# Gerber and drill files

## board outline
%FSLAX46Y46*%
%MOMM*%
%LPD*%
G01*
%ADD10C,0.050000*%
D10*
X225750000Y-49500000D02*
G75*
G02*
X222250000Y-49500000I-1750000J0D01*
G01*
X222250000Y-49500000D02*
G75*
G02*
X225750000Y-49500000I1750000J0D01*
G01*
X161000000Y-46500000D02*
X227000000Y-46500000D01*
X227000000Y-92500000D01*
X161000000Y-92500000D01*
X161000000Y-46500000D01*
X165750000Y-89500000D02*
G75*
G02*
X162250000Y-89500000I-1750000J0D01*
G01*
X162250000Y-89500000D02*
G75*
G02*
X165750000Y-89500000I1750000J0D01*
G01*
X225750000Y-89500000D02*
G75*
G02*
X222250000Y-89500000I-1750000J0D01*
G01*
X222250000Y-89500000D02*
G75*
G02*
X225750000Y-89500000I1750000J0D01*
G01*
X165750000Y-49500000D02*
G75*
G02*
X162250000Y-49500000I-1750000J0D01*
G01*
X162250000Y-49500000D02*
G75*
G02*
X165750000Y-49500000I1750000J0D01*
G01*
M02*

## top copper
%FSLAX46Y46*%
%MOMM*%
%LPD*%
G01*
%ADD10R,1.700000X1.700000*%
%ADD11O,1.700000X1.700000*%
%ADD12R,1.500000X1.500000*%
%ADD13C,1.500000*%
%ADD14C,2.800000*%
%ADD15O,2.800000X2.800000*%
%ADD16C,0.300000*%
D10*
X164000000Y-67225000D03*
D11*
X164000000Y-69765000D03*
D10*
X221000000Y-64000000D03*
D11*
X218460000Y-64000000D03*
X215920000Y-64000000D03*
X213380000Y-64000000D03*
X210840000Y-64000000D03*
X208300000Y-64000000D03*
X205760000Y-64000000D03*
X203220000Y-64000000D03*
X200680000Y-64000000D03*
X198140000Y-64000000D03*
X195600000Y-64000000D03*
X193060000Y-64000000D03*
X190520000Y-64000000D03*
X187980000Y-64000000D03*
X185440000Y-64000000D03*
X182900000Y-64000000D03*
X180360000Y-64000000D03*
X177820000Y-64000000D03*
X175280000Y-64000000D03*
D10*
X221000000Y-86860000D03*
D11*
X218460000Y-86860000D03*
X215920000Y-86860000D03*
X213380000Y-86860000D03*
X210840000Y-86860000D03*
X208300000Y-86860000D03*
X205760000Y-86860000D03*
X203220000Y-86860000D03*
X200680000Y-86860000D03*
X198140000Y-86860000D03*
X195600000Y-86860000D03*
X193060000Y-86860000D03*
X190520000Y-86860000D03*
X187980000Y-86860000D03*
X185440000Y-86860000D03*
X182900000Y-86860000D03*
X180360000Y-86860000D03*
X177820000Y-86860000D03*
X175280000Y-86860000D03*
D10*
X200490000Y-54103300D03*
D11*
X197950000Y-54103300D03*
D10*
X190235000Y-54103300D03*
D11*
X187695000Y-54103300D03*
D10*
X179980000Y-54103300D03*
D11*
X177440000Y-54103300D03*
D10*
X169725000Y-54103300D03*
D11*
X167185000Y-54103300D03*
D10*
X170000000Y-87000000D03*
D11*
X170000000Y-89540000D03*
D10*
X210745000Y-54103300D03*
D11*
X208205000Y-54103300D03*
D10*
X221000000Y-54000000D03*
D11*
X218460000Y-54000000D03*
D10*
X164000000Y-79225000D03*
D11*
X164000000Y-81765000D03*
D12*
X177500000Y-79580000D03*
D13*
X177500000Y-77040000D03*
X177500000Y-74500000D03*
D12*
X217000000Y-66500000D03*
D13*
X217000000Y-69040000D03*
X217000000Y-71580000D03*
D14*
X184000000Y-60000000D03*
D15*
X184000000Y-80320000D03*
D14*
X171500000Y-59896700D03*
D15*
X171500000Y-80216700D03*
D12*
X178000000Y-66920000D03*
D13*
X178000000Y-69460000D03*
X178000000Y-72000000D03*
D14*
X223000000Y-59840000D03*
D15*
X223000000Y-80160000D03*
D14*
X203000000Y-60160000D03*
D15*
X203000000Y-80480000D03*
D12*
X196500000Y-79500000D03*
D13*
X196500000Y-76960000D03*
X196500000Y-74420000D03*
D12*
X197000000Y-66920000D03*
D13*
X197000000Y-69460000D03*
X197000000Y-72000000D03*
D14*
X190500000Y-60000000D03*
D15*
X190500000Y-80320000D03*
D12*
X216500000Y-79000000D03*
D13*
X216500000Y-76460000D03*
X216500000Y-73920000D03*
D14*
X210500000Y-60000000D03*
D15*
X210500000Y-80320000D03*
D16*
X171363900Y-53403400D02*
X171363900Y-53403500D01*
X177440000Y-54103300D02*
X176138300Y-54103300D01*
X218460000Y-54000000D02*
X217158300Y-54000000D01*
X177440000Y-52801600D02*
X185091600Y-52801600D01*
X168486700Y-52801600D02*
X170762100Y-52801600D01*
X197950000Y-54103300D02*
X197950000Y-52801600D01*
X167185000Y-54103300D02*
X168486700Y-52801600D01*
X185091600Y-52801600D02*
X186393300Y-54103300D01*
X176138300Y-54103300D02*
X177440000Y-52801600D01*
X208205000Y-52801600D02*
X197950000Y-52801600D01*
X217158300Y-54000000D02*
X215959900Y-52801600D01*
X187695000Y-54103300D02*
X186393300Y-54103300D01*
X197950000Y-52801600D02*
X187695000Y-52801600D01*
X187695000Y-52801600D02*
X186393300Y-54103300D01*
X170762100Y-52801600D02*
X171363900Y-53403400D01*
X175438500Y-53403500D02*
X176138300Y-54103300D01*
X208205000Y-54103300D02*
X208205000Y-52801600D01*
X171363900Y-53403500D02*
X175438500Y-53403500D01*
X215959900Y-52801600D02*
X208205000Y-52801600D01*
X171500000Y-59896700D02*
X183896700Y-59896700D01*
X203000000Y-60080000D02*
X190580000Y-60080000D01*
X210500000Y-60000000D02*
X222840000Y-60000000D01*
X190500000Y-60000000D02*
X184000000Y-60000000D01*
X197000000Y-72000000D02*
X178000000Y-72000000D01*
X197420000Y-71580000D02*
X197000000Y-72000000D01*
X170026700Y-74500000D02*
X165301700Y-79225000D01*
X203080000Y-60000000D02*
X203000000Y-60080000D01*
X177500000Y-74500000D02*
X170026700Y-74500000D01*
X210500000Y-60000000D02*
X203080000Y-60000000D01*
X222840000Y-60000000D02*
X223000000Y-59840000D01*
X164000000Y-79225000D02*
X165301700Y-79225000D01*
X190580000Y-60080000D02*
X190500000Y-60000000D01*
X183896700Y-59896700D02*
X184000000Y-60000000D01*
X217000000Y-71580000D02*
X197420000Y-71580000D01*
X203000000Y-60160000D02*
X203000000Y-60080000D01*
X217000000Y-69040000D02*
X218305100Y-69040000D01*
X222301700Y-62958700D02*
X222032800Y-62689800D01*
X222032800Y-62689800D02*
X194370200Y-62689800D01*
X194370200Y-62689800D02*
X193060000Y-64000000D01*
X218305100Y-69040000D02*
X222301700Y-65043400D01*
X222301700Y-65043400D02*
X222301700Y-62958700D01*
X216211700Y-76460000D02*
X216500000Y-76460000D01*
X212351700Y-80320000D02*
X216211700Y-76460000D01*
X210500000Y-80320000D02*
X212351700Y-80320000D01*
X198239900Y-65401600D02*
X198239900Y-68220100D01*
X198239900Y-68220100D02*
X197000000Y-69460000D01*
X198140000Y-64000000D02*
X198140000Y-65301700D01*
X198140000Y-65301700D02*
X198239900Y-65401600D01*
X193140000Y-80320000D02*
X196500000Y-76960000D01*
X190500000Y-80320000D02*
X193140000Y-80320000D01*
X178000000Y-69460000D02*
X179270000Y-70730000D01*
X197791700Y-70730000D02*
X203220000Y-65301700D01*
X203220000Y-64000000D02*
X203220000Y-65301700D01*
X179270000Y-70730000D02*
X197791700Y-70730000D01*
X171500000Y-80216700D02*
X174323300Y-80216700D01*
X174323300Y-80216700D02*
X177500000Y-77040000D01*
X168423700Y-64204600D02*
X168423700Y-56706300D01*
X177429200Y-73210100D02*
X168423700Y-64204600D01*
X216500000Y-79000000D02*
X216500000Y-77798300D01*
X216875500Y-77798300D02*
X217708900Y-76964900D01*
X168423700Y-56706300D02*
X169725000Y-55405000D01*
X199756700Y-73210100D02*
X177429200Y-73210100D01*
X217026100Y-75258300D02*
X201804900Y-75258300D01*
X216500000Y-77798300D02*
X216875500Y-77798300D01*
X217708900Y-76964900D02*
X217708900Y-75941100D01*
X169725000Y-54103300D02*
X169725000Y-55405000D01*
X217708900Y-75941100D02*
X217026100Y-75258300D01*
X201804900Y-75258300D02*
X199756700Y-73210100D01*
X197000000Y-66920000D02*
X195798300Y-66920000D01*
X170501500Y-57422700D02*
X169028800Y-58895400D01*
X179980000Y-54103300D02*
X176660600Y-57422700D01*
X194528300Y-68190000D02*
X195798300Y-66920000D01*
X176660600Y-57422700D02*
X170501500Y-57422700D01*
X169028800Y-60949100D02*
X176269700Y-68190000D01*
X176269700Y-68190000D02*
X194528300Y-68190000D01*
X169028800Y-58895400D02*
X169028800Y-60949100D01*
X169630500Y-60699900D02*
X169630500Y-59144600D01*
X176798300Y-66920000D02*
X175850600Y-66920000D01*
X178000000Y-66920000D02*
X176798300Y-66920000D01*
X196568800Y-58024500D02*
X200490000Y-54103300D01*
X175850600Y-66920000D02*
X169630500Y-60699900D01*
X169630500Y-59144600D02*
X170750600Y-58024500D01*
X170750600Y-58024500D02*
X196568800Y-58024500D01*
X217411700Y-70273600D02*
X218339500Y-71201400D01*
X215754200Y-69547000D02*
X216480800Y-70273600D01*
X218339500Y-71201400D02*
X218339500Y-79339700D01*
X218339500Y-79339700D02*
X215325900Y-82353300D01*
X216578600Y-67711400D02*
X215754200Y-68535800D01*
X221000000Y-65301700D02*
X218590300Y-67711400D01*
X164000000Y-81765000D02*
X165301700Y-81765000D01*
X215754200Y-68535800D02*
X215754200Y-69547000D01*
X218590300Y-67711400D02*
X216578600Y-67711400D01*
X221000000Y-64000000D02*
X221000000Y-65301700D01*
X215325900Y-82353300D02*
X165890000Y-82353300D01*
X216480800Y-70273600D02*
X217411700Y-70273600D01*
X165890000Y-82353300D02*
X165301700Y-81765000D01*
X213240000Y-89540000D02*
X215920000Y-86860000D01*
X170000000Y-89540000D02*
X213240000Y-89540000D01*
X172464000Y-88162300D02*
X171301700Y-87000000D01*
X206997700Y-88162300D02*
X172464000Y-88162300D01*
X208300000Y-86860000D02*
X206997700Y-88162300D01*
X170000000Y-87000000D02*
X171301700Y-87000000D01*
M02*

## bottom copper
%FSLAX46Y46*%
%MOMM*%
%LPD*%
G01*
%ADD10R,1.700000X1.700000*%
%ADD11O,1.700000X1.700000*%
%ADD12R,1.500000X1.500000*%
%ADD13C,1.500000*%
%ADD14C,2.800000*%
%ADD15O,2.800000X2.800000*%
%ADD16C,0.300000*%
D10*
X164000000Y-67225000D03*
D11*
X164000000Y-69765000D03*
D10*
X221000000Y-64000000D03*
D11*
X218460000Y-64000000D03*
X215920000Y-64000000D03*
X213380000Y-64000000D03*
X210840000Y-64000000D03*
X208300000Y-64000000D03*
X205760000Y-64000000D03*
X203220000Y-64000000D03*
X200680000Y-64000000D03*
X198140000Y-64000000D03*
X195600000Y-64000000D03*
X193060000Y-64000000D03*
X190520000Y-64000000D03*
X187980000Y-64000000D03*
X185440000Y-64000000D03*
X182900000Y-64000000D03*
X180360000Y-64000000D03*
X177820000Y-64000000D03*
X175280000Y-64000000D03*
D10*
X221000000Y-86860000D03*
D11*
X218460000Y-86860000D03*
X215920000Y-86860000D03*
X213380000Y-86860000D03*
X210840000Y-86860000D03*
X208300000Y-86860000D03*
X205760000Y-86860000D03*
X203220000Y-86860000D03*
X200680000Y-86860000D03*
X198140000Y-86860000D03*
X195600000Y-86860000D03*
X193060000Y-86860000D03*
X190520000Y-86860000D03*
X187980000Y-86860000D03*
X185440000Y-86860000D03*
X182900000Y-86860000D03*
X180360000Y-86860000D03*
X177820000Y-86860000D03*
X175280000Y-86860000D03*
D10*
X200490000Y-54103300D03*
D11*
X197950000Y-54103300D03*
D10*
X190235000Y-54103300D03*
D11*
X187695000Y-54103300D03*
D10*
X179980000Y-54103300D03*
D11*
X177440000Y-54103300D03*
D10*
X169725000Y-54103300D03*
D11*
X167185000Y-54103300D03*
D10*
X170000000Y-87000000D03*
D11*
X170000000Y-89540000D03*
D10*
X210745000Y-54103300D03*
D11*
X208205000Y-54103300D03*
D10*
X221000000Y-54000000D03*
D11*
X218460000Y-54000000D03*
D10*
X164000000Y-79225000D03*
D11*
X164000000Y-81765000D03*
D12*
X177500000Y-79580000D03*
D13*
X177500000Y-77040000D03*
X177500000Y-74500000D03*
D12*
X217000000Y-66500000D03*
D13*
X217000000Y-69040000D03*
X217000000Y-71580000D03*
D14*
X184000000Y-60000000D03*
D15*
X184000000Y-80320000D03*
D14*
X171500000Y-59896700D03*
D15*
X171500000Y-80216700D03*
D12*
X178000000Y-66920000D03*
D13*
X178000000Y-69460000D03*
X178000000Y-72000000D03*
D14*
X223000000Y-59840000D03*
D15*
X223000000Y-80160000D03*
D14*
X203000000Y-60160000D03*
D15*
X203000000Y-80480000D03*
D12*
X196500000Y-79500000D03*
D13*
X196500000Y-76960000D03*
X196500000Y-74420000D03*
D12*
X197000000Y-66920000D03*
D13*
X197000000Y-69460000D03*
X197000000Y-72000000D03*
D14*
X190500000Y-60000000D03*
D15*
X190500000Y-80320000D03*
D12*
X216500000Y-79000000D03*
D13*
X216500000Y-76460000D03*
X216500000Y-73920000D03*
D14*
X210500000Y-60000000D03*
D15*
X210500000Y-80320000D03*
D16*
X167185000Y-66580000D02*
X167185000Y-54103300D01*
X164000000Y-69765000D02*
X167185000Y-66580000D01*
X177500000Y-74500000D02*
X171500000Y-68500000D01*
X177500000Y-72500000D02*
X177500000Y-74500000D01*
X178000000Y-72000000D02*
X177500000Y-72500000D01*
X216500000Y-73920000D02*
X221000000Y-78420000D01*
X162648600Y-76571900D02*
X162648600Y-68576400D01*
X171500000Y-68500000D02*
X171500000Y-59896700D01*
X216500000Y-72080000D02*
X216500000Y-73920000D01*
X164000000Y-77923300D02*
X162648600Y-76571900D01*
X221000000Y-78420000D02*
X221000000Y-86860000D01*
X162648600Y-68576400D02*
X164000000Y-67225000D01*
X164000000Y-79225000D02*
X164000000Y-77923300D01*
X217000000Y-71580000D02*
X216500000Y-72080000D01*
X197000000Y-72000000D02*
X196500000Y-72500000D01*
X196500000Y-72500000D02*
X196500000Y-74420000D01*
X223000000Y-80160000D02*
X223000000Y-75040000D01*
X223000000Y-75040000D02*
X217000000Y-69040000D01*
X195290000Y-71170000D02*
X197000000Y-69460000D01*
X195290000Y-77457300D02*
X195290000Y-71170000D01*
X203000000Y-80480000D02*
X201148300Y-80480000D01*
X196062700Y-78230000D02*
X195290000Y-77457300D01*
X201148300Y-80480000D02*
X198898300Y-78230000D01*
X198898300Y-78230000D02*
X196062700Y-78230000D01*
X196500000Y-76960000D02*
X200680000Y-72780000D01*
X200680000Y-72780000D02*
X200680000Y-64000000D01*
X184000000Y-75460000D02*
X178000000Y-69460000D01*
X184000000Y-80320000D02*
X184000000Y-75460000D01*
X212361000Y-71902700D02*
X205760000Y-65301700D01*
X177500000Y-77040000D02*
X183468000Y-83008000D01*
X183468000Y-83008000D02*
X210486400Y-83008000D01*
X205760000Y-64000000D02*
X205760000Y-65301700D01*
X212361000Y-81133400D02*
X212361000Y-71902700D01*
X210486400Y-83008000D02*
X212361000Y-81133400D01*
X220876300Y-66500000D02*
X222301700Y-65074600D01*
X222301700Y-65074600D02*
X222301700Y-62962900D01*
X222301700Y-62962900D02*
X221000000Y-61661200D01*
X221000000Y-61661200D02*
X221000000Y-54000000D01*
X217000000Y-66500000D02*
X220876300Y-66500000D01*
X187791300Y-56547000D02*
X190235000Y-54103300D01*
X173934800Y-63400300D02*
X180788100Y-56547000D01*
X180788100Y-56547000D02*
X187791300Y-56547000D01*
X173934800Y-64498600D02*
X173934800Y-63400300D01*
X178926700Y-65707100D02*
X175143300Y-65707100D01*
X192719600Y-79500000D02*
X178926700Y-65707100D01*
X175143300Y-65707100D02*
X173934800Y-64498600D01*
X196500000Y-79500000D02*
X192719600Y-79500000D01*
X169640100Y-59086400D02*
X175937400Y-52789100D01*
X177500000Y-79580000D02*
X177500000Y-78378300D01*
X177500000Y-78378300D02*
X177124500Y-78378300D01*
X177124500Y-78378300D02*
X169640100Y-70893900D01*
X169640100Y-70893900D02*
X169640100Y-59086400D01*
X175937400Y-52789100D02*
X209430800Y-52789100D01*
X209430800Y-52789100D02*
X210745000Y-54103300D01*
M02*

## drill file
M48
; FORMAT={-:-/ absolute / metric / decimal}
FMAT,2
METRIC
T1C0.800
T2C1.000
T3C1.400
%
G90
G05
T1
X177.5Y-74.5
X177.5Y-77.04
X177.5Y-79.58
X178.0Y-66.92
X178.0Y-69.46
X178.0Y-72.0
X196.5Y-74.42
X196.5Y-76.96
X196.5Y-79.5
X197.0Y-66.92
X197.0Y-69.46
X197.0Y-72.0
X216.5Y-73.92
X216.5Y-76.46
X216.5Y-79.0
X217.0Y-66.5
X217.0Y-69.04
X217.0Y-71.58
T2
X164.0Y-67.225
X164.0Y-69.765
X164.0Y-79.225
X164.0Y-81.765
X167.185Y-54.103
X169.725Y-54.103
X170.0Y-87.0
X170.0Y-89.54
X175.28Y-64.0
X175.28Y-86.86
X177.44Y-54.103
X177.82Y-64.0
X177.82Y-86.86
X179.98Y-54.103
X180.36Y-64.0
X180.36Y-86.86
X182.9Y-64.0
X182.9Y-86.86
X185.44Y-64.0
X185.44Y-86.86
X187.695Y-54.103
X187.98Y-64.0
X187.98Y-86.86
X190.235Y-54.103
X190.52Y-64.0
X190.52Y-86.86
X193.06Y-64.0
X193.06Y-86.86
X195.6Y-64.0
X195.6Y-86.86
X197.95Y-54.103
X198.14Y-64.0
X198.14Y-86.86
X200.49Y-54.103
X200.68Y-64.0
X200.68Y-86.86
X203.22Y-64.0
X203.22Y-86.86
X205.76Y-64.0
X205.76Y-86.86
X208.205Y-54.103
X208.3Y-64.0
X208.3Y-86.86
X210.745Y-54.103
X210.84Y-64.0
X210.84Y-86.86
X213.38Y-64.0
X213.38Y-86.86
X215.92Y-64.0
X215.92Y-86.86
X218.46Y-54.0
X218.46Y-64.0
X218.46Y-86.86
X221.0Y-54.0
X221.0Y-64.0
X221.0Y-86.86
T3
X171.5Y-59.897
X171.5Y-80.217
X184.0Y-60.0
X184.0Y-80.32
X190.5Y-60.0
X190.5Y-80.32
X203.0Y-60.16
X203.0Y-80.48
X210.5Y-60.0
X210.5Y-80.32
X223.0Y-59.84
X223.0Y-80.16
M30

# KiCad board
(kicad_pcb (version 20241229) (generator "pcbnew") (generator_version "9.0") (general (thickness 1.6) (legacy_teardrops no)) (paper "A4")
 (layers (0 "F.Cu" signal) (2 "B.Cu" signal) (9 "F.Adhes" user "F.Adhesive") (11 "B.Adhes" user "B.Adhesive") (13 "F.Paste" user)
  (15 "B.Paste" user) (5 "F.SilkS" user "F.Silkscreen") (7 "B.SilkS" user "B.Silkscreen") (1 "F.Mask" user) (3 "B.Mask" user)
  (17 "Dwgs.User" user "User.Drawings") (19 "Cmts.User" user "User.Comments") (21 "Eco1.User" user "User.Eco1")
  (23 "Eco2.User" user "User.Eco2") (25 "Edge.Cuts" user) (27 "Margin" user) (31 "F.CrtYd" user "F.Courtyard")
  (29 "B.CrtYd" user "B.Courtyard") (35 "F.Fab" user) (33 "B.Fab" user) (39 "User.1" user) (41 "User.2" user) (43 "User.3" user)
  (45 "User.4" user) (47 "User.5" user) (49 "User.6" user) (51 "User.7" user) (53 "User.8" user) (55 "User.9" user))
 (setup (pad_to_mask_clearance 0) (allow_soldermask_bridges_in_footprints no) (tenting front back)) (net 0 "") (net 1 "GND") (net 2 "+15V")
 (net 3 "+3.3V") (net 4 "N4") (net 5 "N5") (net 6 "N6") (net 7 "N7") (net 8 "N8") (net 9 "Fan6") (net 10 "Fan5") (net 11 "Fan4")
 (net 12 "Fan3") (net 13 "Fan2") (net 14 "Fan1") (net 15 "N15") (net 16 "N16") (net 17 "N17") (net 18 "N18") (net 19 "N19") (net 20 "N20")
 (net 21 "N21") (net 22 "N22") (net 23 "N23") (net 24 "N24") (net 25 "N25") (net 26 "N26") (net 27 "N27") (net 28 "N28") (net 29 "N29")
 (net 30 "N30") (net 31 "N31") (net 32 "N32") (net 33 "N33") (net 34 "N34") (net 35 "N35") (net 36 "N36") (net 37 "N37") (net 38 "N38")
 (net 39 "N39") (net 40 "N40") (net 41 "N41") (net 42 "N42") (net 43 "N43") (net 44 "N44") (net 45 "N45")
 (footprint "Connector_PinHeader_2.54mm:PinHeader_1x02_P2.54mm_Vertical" (layer "F.Cu") (at 164 67.225)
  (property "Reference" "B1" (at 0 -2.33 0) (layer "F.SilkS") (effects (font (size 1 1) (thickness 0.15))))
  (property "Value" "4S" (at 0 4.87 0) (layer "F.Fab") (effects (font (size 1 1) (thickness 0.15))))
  (pad "1" thru_hole rect (at 0 0) (size 1.7 1.7) (drill 1) (layers "*.Cu" "*.Mask") (remove_unused_layers no) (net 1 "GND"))
  (pad "2" thru_hole oval (at 0 2.54) (size 1.7 1.7) (drill 1) (layers "*.Cu" "*.Mask") (remove_unused_layers no) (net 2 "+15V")))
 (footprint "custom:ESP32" (layer "F.Cu") (at 221 75.43 -90)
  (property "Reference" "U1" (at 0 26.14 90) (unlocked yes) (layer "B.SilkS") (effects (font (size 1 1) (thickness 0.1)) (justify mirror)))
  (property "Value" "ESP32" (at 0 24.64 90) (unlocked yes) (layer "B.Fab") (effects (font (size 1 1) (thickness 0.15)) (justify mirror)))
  (pad "1" thru_hole rect (at -11.43 0 270) (size 1.7 1.7) (drill 1) (layers "*.Cu" "*.Mask") (remove_unused_layers no) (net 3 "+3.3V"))
  (pad "2" thru_hole oval (at -11.43 2.54 270) (size 1.7 1.7) (drill 1) (layers "*.Cu" "*.Mask") (remove_unused_layers no) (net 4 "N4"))
  (pad "3" thru_hole oval (at -11.43 5.08 270) (size 1.7 1.7) (drill 1) (layers "*.Cu" "*.Mask") (remove_unused_layers no) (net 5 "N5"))
  (pad "4" thru_hole oval (at -11.43 7.62 270) (size 1.7 1.7) (drill 1) (layers "*.Cu" "*.Mask") (remove_unused_layers no) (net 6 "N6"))
  (pad "5" thru_hole oval (at -11.43 10.16 270) (size 1.7 1.7) (drill 1) (layers "*.Cu" "*.Mask") (remove_unused_layers no) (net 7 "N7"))
  (pad "6" thru_hole oval (at -11.43 12.7 270) (size 1.7 1.7) (drill 1) (layers "*.Cu" "*.Mask") (remove_unused_layers no) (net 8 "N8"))
  (pad "7" thru_hole oval (at -11.43 15.24 270) (size 1.7 1.7) (drill 1) (layers "*.Cu" "*.Mask") (remove_unused_layers no) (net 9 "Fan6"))
  (pad "8" thru_hole oval (at -11.43 17.78 270) (size 1.7 1.7) (drill 1) (layers "*.Cu" "*.Mask") (remove_unused_layers no) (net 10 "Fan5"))
  (pad "9" thru_hole oval (at -11.43 20.32 270) (size 1.7 1.7) (drill 1) (layers "*.Cu" "*.Mask") (remove_unused_layers no) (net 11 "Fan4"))
  (pad "10" thru_hole oval (at -11.43 22.86 270) (size 1.7 1.7) (drill 1) (layers "*.Cu" "*.Mask") (remove_unused_layers no) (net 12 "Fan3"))
  (pad "11" thru_hole oval (at -11.43 25.4 270) (size 1.7 1.7) (drill 1) (layers "*.Cu" "*.Mask") (remove_unused_layers no) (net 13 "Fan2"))
  (pad "12" thru_hole oval (at -11.43 27.94 270) (size 1.7 1.7) (drill 1) (layers "*.Cu" "*.Mask") (remove_unused_layers no) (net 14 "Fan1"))
  (pad "13" thru_hole oval (at -11.43 30.48 270) (size 1.7 1.7) (drill 1) (layers "*.Cu" "*.Mask") (remove_unused_layers no) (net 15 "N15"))
  (pad "14" thru_hole oval (at -11.43 33.02 270) (size 1.7 1.7) (drill 1) (layers "*.Cu" "*.Mask") (remove_unused_layers no) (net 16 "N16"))
  (pad "15" thru_hole oval (at -11.43 35.56 270) (size 1.7 1.7) (drill 1) (layers "*.Cu" "*.Mask") (remove_unused_layers no) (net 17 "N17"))
  (pad "16" thru_hole oval (at -11.43 38.1 270) (size 1.7 1.7) (drill 1) (layers "*.Cu" "*.Mask") (remove_unused_layers no) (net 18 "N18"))
  (pad "17" thru_hole oval (at -11.43 40.64 270) (size 1.7 1.7) (drill 1) (layers "*.Cu" "*.Mask") (remove_unused_layers no) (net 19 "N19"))
  (pad "18" thru_hole oval (at -11.43 43.18 270) (size 1.7 1.7) (drill 1) (layers "*.Cu" "*.Mask") (remove_unused_layers no) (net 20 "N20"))
  (pad "19" thru_hole oval (at -11.43 45.72 270) (size 1.7 1.7) (drill 1) (layers "*.Cu" "*.Mask") (remove_unused_layers no) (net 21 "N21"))
  (pad "20" thru_hole rect (at 11.43 0 270) (size 1.7 1.7) (drill 1) (layers "*.Cu" "*.Mask") (remove_unused_layers no) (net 1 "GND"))
  (pad "21" thru_hole oval (at 11.43 2.54 270) (size 1.7 1.7) (drill 1) (layers "*.Cu" "*.Mask") (remove_unused_layers no) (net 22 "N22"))
  (pad "22" thru_hole oval (at 11.43 5.08 270) (size 1.7 1.7) (drill 1) (layers "*.Cu" "*.Mask") (remove_unused_layers no) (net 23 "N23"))
  (pad "23" thru_hole oval (at 11.43 7.62 270) (size 1.7 1.7) (drill 1) (layers "*.Cu" "*.Mask") (remove_unused_layers no) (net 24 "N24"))
  (pad "24" thru_hole oval (at 11.43 10.16 270) (size 1.7 1.7) (drill 1) (layers "*.Cu" "*.Mask") (remove_unused_layers no) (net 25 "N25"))
  (pad "25" thru_hole oval (at 11.43 12.7 270) (size 1.7 1.7) (drill 1) (layers "*.Cu" "*.Mask") (remove_unused_layers no) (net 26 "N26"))
  (pad "26" thru_hole oval (at 11.43 15.24 270) (size 1.7 1.7) (drill 1) (layers "*.Cu" "*.Mask") (remove_unused_layers no) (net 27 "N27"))
  (pad "27" thru_hole oval (at 11.43 17.78 270) (size 1.7 1.7) (drill 1) (layers "*.Cu" "*.Mask") (remove_unused_layers no) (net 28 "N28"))
  (pad "28" thru_hole oval (at 11.43 20.32 270) (size 1.7 1.7) (drill 1) (layers "*.Cu" "*.Mask") (remove_unused_layers no) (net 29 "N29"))
  (pad "29" thru_hole oval (at 11.43 22.86 270) (size 1.7 1.7) (drill 1) (layers "*.Cu" "*.Mask") (remove_unused_layers no) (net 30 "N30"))
  (pad "30" thru_hole oval (at 11.43 25.4 270) (size 1.7 1.7) (drill 1) (layers "*.Cu" "*.Mask") (remove_unused_layers no) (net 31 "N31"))
  (pad "31" thru_hole oval (at 11.43 27.94 270) (size 1.7 1.7) (drill 1) (layers "*.Cu" "*.Mask") (remove_unused_layers no) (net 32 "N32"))
  (pad "32" thru_hole oval (at 11.43 30.48 270) (size 1.7 1.7) (drill 1) (layers "*.Cu" "*.Mask") (remove_unused_layers no) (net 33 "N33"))
  (pad "33" thru_hole oval (at 11.43 33.02 270) (size 1.7 1.7) (drill 1) (layers "*.Cu" "*.Mask") (remove_unused_layers no) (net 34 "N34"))
  (pad "34" thru_hole oval (at 11.43 35.56 270) (size 1.7 1.7) (drill 1) (layers "*.Cu" "*.Mask") (remove_unused_layers no) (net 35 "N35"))
  (pad "35" thru_hole oval (at 11.43 38.1 270) (size 1.7 1.7) (drill 1) (layers "*.Cu" "*.Mask") (remove_unused_layers no) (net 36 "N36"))
  (pad "36" thru_hole oval (at 11.43 40.64 270) (size 1.7 1.7) (drill 1) (layers "*.Cu" "*.Mask") (remove_unused_layers no) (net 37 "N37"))
  (pad "37" thru_hole oval (at 11.43 43.18 270) (size 1.7 1.7) (drill 1) (layers "*.Cu" "*.Mask") (remove_unused_layers no) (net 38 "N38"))
  (pad "38" thru_hole oval (at 11.43 45.72 270) (size 1.7 1.7) (drill 1) (layers "*.Cu" "*.Mask") (remove_unused_layers no) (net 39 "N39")))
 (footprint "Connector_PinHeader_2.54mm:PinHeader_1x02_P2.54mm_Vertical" (layer "F.Cu") (at 200.49 54.1033 -90)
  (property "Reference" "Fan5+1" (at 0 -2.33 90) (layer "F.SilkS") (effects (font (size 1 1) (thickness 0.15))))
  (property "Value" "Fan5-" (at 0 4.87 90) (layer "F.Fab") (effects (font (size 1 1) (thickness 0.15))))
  (pad "1" thru_hole rect (at 0 0 270) (size 1.7 1.7) (drill 1) (layers "*.Cu" "*.Mask") (remove_unused_layers no) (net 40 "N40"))
  (pad "2" thru_hole oval (at 0 2.54 270) (size 1.7 1.7) (drill 1) (layers "*.Cu" "*.Mask") (remove_unused_layers no) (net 2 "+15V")))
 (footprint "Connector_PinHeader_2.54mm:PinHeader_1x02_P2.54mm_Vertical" (layer "F.Cu") (at 190.235 54.1033 -90)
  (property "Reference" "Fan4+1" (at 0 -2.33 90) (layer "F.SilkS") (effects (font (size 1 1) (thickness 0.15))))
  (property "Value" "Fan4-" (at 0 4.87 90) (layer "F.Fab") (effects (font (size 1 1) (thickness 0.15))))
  (pad "1" thru_hole rect (at 0 0 270) (size 1.7 1.7) (drill 1) (layers "*.Cu" "*.Mask") (remove_unused_layers no) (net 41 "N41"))
  (pad "2" thru_hole oval (at 0 2.54 270) (size 1.7 1.7) (drill 1) (layers "*.Cu" "*.Mask") (remove_unused_layers no) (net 2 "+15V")))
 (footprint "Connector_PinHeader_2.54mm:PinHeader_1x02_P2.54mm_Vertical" (layer "F.Cu") (at 179.98 54.1033 -90)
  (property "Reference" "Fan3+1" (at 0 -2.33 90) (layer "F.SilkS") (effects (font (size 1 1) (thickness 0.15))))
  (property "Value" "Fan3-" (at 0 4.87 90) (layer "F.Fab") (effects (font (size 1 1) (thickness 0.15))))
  (pad "1" thru_hole rect (at 0 0 270) (size 1.7 1.7) (drill 1) (layers "*.Cu" "*.Mask") (remove_unused_layers no) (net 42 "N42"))
  (pad "2" thru_hole oval (at 0 2.54 270) (size 1.7 1.7) (drill 1) (layers "*.Cu" "*.Mask") (remove_unused_layers no) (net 2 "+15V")))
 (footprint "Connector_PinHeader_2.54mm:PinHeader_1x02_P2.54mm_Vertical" (layer "F.Cu") (at 169.725 54.1033 -90)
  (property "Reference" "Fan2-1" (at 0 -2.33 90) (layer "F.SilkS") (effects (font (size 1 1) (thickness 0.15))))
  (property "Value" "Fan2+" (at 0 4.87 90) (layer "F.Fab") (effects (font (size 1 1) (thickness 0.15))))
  (pad "1" thru_hole rect (at 0 0 270) (size 1.7 1.7) (drill 1) (layers "*.Cu" "*.Mask") (remove_unused_layers no) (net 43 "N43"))
  (pad "2" thru_hole oval (at 0 2.54 270) (size 1.7 1.7) (drill 1) (layers "*.Cu" "*.Mask") (remove_unused_layers no) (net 2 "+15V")))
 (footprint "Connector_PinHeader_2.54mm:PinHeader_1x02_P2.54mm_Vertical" (layer "F.Cu") (at 170 87)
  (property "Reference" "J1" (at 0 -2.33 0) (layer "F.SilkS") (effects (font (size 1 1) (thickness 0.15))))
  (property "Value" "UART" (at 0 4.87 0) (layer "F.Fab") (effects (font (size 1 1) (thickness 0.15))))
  (pad "1" thru_hole rect (at 0 0) (size 1.7 1.7) (drill 1) (layers "*.Cu" "*.Mask") (remove_unused_layers no) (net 26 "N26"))
  (pad "2" thru_hole oval (at 0 2.54) (size 1.7 1.7) (drill 1) (layers "*.Cu" "*.Mask") (remove_unused_layers no) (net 23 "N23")))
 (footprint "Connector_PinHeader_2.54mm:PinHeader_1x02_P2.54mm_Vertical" (layer "F.Cu") (at 210.745 54.1033 -90)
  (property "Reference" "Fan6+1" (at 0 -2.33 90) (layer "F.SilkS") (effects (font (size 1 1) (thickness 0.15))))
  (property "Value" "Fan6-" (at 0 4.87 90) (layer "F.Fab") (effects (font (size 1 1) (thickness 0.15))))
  (pad "1" thru_hole rect (at 0 0 270) (size 1.7 1.7) (drill 1) (layers "*.Cu" "*.Mask") (remove_unused_layers no) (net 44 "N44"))
  (pad "2" thru_hole oval (at 0 2.54 270) (size 1.7 1.7) (drill 1) (layers "*.Cu" "*.Mask") (remove_unused_layers no) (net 2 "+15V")))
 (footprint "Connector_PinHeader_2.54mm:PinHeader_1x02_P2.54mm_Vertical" (layer "F.Cu") (at 221 54 -90)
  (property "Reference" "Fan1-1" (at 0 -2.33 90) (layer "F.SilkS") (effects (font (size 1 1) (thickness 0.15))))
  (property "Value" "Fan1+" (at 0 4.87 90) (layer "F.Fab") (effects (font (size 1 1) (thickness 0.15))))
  (pad "1" thru_hole rect (at 0 0 270) (size 1.7 1.7) (drill 1) (layers "*.Cu" "*.Mask") (remove_unused_layers no) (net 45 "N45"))
  (pad "2" thru_hole oval (at 0 2.54 270) (size 1.7 1.7) (drill 1) (layers "*.Cu" "*.Mask") (remove_unused_layers no) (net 2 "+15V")))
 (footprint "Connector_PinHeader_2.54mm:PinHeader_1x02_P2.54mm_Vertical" (layer "F.Cu") (at 164 79.225)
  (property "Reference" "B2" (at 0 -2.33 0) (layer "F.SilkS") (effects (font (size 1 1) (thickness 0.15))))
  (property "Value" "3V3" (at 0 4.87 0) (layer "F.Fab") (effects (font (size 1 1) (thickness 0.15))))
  (pad "1" thru_hole rect (at 0 0) (size 1.7 1.7) (drill 1) (layers "*.Cu" "*.Mask") (remove_unused_layers no) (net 1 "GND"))
  (pad "2" thru_hole oval (at 0 2.54) (size 1.7 1.7) (drill 1) (layers "*.Cu" "*.Mask") (remove_unused_layers no) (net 3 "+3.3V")))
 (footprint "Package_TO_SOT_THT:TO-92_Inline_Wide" (layer "B.Cu") (at 177.5 79.58 90)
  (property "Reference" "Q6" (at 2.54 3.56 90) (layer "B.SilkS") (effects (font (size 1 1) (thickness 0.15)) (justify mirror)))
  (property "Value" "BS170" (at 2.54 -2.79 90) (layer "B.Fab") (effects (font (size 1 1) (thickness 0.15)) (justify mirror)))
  (pad "1" thru_hole rect (at 0 0 90) (size 1.5 1.5) (drill 0.8) (layers "*.Cu" "*.Mask") (remove_unused_layers no) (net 44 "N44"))
  (pad "2" thru_hole circle (at 2.54 0 90) (size 1.5 1.5) (drill 0.8) (layers "*.Cu" "*.Mask") (remove_unused_layers no) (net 9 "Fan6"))
  (pad "3" thru_hole circle (at 5.08 0 90) (size 1.5 1.5) (drill 0.8) (layers "*.Cu" "*.Mask") (remove_unused_layers no) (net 1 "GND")))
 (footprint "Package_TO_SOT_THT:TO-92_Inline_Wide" (layer "B.Cu") (at 217 66.5 -90)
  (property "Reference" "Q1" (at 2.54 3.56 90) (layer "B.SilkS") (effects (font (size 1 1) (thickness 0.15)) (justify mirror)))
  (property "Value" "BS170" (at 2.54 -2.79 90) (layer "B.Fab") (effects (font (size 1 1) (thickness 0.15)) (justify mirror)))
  (pad "1" thru_hole rect (at 0 0 270) (size 1.5 1.5) (drill 0.8) (layers "*.Cu" "*.Mask") (remove_unused_layers no) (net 45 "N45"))
  (pad "2" thru_hole circle (at 2.54 0 270) (size 1.5 1.5) (drill 0.8) (layers "*.Cu" "*.Mask") (remove_unused_layers no) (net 14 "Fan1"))
  (pad "3" thru_hole circle (at 5.08 0 270) (size 1.5 1.5) (drill 0.8) (layers "*.Cu" "*.Mask") (remove_unused_layers no) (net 1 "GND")))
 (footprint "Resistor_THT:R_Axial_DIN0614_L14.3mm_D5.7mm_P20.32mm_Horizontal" (layer "B.Cu") (at 184 60 -90)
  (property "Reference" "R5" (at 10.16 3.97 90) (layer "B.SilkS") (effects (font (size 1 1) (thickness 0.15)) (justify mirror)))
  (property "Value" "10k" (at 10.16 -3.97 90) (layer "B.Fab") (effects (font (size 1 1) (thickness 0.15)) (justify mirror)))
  (pad "1" thru_hole circle (at 0 0 270) (size 2.8 2.8) (drill 1.4) (layers "*.Cu" "*.Mask") (remove_unused_layers no) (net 1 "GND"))
  (pad "2" thru_hole oval (at 20.32 0 270) (size 2.8 2.8) (drill 1.4) (layers "*.Cu" "*.Mask") (remove_unused_layers no) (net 10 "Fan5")))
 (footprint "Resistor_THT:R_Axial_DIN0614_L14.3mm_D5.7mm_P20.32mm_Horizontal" (layer "B.Cu") (at 171.5 59.8967 -90)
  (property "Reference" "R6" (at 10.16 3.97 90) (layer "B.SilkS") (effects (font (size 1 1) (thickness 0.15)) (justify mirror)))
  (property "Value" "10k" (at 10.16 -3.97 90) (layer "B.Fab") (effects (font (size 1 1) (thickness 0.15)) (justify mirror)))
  (pad "1" thru_hole circle (at 0 0 270) (size 2.8 2.8) (drill 1.4) (layers "*.Cu" "*.Mask") (remove_unused_layers no) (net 1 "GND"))
  (pad "2" thru_hole oval (at 20.32 0 270) (size 2.8 2.8) (drill 1.4) (layers "*.Cu" "*.Mask") (remove_unused_layers no) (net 9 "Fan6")))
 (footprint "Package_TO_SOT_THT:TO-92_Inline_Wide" (layer "B.Cu") (at 178 66.92 -90)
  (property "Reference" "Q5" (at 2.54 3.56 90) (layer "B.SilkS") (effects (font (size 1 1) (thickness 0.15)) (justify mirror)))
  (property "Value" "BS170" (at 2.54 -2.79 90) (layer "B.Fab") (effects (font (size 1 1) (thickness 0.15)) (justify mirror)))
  (pad "1" thru_hole rect (at 0 0 270) (size 1.5 1.5) (drill 0.8) (layers "*.Cu" "*.Mask") (remove_unused_layers no) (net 40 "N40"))
  (pad "2" thru_hole circle (at 2.54 0 270) (size 1.5 1.5) (drill 0.8) (layers "*.Cu" "*.Mask") (remove_unused_layers no) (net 10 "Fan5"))
  (pad "3" thru_hole circle (at 5.08 0 270) (size 1.5 1.5) (drill 0.8) (layers "*.Cu" "*.Mask") (remove_unused_layers no) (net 1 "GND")))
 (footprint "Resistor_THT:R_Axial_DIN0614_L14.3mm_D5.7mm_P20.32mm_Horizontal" (layer "B.Cu") (at 223 59.84 -90)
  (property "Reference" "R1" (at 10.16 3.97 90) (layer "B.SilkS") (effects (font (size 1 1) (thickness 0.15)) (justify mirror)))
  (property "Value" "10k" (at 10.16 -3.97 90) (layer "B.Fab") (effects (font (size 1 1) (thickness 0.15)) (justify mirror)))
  (pad "1" thru_hole circle (at 0 0 270) (size 2.8 2.8) (drill 1.4) (layers "*.Cu" "*.Mask") (remove_unused_layers no) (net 1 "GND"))
  (pad "2" thru_hole oval (at 20.32 0 270) (size 2.8 2.8) (drill 1.4) (layers "*.Cu" "*.Mask") (remove_unused_layers no) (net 14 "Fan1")))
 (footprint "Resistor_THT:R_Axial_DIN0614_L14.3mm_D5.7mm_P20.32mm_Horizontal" (layer "B.Cu") (at 203 60.16 -90)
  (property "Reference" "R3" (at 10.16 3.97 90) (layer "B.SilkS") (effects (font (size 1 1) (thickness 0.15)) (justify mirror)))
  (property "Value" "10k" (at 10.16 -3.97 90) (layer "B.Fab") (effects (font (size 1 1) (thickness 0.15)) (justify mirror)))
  (pad "1" thru_hole circle (at 0 0 270) (size 2.8 2.8) (drill 1.4) (layers "*.Cu" "*.Mask") (remove_unused_layers no) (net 1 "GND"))
  (pad "2" thru_hole oval (at 20.32 0 270) (size 2.8 2.8) (drill 1.4) (layers "*.Cu" "*.Mask") (remove_unused_layers no) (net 12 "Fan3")))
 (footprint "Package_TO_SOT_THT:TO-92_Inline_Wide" (layer "B.Cu") (at 196.5 79.5 90)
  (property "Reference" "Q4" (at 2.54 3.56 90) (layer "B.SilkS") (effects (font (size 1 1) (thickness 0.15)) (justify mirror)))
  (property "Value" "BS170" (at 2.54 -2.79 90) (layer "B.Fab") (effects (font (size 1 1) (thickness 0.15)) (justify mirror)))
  (pad "1" thru_hole rect (at 0 0 90) (size 1.5 1.5) (drill 0.8) (layers "*.Cu" "*.Mask") (remove_unused_layers no) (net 41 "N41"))
  (pad "2" thru_hole circle (at 2.54 0 90) (size 1.5 1.5) (drill 0.8) (layers "*.Cu" "*.Mask") (remove_unused_layers no) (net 11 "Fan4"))
  (pad "3" thru_hole circle (at 5.08 0 90) (size 1.5 1.5) (drill 0.8) (layers "*.Cu" "*.Mask") (remove_unused_layers no) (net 1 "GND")))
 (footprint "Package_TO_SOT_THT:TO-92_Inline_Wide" (layer "B.Cu") (at 197 66.92 -90)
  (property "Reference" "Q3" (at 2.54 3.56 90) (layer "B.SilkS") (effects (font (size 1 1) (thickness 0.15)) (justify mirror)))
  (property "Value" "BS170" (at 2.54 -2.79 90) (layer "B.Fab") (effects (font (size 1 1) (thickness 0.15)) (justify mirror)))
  (pad "1" thru_hole rect (at 0 0 270) (size 1.5 1.5) (drill 0.8) (layers "*.Cu" "*.Mask") (remove_unused_layers no) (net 42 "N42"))
  (pad "2" thru_hole circle (at 2.54 0 270) (size 1.5 1.5) (drill 0.8) (layers "*.Cu" "*.Mask") (remove_unused_layers no) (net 12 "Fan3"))
  (pad "3" thru_hole circle (at 5.08 0 270) (size 1.5 1.5) (drill 0.8) (layers "*.Cu" "*.Mask") (remove_unused_layers no) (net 1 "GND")))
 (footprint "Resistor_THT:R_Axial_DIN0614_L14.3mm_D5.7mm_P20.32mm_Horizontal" (layer "B.Cu") (at 190.5 60 -90)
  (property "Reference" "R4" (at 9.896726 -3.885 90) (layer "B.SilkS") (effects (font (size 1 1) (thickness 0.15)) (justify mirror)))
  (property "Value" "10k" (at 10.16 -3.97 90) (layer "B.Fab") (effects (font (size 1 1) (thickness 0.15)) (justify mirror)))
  (pad "1" thru_hole circle (at 0 0 270) (size 2.8 2.8) (drill 1.4) (layers "*.Cu" "*.Mask") (remove_unused_layers no) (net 1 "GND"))
  (pad "2" thru_hole oval (at 20.32 0 270) (size 2.8 2.8) (drill 1.4) (layers "*.Cu" "*.Mask") (remove_unused_layers no) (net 11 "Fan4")))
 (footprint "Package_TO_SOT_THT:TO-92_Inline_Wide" (layer "B.Cu") (at 216.5 79 90)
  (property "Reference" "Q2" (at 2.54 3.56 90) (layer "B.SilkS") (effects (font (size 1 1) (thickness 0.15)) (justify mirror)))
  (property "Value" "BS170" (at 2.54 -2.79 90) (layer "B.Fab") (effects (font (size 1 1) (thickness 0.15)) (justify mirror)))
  (pad "1" thru_hole rect (at 0 0 90) (size 1.5 1.5) (drill 0.8) (layers "*.Cu" "*.Mask") (remove_unused_layers no) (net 43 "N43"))
  (pad "2" thru_hole circle (at 2.54 0 90) (size 1.5 1.5) (drill 0.8) (layers "*.Cu" "*.Mask") (remove_unused_layers no) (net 13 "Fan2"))
  (pad "3" thru_hole circle (at 5.08 0 90) (size 1.5 1.5) (drill 0.8) (layers "*.Cu" "*.Mask") (remove_unused_layers no) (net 1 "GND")))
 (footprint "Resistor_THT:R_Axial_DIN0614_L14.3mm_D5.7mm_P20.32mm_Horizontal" (layer "B.Cu") (at 210.5 60 -90)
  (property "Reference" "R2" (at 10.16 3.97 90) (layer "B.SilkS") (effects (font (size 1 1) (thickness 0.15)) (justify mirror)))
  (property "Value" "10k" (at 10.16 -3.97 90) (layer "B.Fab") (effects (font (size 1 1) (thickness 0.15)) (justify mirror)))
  (pad "1" thru_hole circle (at 0 0 270) (size 2.8 2.8) (drill 1.4) (layers "*.Cu" "*.Mask") (remove_unused_layers no) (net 1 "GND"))
  (pad "2" thru_hole oval (at 20.32 0 270) (size 2.8 2.8) (drill 1.4) (layers "*.Cu" "*.Mask") (remove_unused_layers no) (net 13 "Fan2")))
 (gr_circle (center 224 49.5) (end 225.75 49.5) (stroke (width 0.05) (type solid)) (fill no) (layer "Edge.Cuts"))
 (gr_rect (start 161 46.5) (end 227 92.5) (stroke (width 0.05) (type default)) (fill no) (layer "Edge.Cuts"))
 (gr_circle (center 164 89.5) (end 165.75 89.5) (stroke (width 0.05) (type solid)) (fill no) (layer "Edge.Cuts"))
 (gr_circle (center 224 89.5) (end 225.75 89.5) (stroke (width 0.05) (type solid)) (fill no) (layer "Edge.Cuts"))
 (gr_circle (center 164 49.5) (end 165.75 49.5) (stroke (width 0.05) (type solid)) (fill no) (layer "Edge.Cuts"))
 (segment (start 171.3639 53.4034) (end 171.3639 53.4035) (width 0.3) (layer "F.Cu") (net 2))
 (segment (start 177.44 54.1033) (end 176.1383 54.1033) (width 0.3) (layer "F.Cu") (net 2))
 (segment (start 218.46 54) (end 217.1583 54) (width 0.3) (layer "F.Cu") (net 2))
 (segment (start 177.44 52.8016) (end 185.0916 52.8016) (width 0.3) (layer "F.Cu") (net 2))
 (segment (start 168.4867 52.8016) (end 170.7621 52.8016) (width 0.3) (layer "F.Cu") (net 2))
 (segment (start 197.95 54.1033) (end 197.95 52.8016) (width 0.3) (layer "F.Cu") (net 2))
 (segment (start 167.185 54.1033) (end 168.4867 52.8016) (width 0.3) (layer "F.Cu") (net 2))
 (segment (start 185.0916 52.8016) (end 186.3933 54.1033) (width 0.3) (layer "F.Cu") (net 2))
 (segment (start 176.1383 54.1033) (end 177.44 52.8016) (width 0.3) (layer "F.Cu") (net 2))
 (segment (start 208.205 52.8016) (end 197.95 52.8016) (width 0.3) (layer "F.Cu") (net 2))
 (segment (start 217.1583 54) (end 215.9599 52.8016) (width 0.3) (layer "F.Cu") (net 2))
 (segment (start 187.695 54.1033) (end 186.3933 54.1033) (width 0.3) (layer "F.Cu") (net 2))
 (segment (start 197.95 52.8016) (end 187.695 52.8016) (width 0.3) (layer "F.Cu") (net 2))
 (segment (start 187.695 52.8016) (end 186.3933 54.1033) (width 0.3) (layer "F.Cu") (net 2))
 (segment (start 170.7621 52.8016) (end 171.3639 53.4034) (width 0.3) (layer "F.Cu") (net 2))
 (segment (start 175.4385 53.4035) (end 176.1383 54.1033) (width 0.3) (layer "F.Cu") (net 2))
 (segment (start 208.205 54.1033) (end 208.205 52.8016) (width 0.3) (layer "F.Cu") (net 2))
 (segment (start 171.3639 53.4035) (end 175.4385 53.4035) (width 0.3) (layer "F.Cu") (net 2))
 (segment (start 215.9599 52.8016) (end 208.205 52.8016) (width 0.3) (layer "F.Cu") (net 2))
 (segment (start 167.185 66.58) (end 167.185 54.1033) (width 0.3) (layer "B.Cu") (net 2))
 (segment (start 164 69.765) (end 167.185 66.58) (width 0.3) (layer "B.Cu") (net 2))
 (segment (start 171.5 59.8967) (end 183.8967 59.8967) (width 0.3) (layer "F.Cu") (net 1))
 (segment (start 203 60.08) (end 190.58 60.08) (width 0.3) (layer "F.Cu") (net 1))
 (segment (start 210.5 60) (end 222.84 60) (width 0.3) (layer "F.Cu") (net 1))
 (segment (start 190.5 60) (end 184 60) (width 0.3) (layer "F.Cu") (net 1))
 (segment (start 197 72) (end 178 72) (width 0.3) (layer "F.Cu") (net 1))
 (segment (start 197.42 71.58) (end 197 72) (width 0.3) (layer "F.Cu") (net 1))
 (segment (start 170.0267 74.5) (end 165.3017 79.225) (width 0.3) (layer "F.Cu") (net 1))
 (segment (start 203.08 60) (end 203 60.08) (width 0.3) (layer "F.Cu") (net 1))
 (segment (start 177.5 74.5) (end 170.0267 74.5) (width 0.3) (layer "F.Cu") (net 1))
 (segment (start 210.5 60) (end 203.08 60) (width 0.3) (layer "F.Cu") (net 1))
 (segment (start 222.84 60) (end 223 59.84) (width 0.3) (layer "F.Cu") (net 1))
 (segment (start 164 79.225) (end 165.3017 79.225) (width 0.3) (layer "F.Cu") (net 1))
 (segment (start 190.58 60.08) (end 190.5 60) (width 0.3) (layer "F.Cu") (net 1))
 (segment (start 183.8967 59.8967) (end 184 60) (width 0.3) (layer "F.Cu") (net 1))
 (segment (start 217 71.58) (end 197.42 71.58) (width 0.3) (layer "F.Cu") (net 1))
 (segment (start 203 60.16) (end 203 60.08) (width 0.3) (layer "F.Cu") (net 1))
 (segment (start 177.5 74.5) (end 171.5 68.5) (width 0.3) (layer "B.Cu") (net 1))
 (segment (start 177.5 72.5) (end 177.5 74.5) (width 0.3) (layer "B.Cu") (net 1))
 (segment (start 178 72) (end 177.5 72.5) (width 0.3) (layer "B.Cu") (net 1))
 (segment (start 216.5 73.92) (end 221 78.42) (width 0.3) (layer "B.Cu") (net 1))
 (segment (start 162.6486 76.5719) (end 162.6486 68.5764) (width 0.3) (layer "B.Cu") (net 1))
 (segment (start 171.5 68.5) (end 171.5 59.8967) (width 0.3) (layer "B.Cu") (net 1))
 (segment (start 216.5 72.08) (end 216.5 73.92) (width 0.3) (layer "B.Cu") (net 1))
 (segment (start 164 77.9233) (end 162.6486 76.5719) (width 0.3) (layer "B.Cu") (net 1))
 (segment (start 221 78.42) (end 221 86.86) (width 0.3) (layer "B.Cu") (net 1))
 (segment (start 162.6486 68.5764) (end 164 67.225) (width 0.3) (layer "B.Cu") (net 1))
 (segment (start 164 79.225) (end 164 77.9233) (width 0.3) (layer "B.Cu") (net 1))
 (segment (start 217 71.58) (end 216.5 72.08) (width 0.3) (layer "B.Cu") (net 1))
 (segment (start 197 72) (end 196.5 72.5) (width 0.3) (layer "B.Cu") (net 1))
 (segment (start 196.5 72.5) (end 196.5 74.42) (width 0.3) (layer "B.Cu") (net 1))
 (segment (start 217 69.04) (end 218.3051 69.04) (width 0.3) (layer "F.Cu") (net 14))
 (segment (start 222.3017 62.9587) (end 222.0328 62.6898) (width 0.3) (layer "F.Cu") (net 14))
 (segment (start 222.0328 62.6898) (end 194.3702 62.6898) (width 0.3) (layer "F.Cu") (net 14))
 (segment (start 194.3702 62.6898) (end 193.06 64) (width 0.3) (layer "F.Cu") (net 14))
 (segment (start 218.3051 69.04) (end 222.3017 65.0434) (width 0.3) (layer "F.Cu") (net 14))
 (segment (start 222.3017 65.0434) (end 222.3017 62.9587) (width 0.3) (layer "F.Cu") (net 14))
 (segment (start 223 80.16) (end 223 75.04) (width 0.3) (layer "B.Cu") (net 14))
 (segment (start 223 75.04) (end 217 69.04) (width 0.3) (layer "B.Cu") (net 14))
 (segment (start 216.2117 76.46) (end 216.5 76.46) (width 0.3) (layer "F.Cu") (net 13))
 (segment (start 212.3517 80.32) (end 216.2117 76.46) (width 0.3) (layer "F.Cu") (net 13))
 (segment (start 210.5 80.32) (end 212.3517 80.32) (width 0.3) (layer "F.Cu") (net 13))
 (segment (start 198.2399 65.4016) (end 198.2399 68.2201) (width 0.3) (layer "F.Cu") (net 12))
 (segment (start 198.2399 68.2201) (end 197 69.46) (width 0.3) (layer "F.Cu") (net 12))
 (segment (start 198.14 64) (end 198.14 65.3017) (width 0.3) (layer "F.Cu") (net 12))
 (segment (start 198.14 65.3017) (end 198.2399 65.4016) (width 0.3) (layer "F.Cu") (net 12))
 (segment (start 195.29 71.17) (end 197 69.46) (width 0.3) (layer "B.Cu") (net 12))
 (segment (start 195.29 77.4573) (end 195.29 71.17) (width 0.3) (layer "B.Cu") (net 12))
 (segment (start 203 80.48) (end 201.1483 80.48) (width 0.3) (layer "B.Cu") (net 12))
 (segment (start 196.0627 78.23) (end 195.29 77.4573) (width 0.3) (layer "B.Cu") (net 12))
 (segment (start 201.1483 80.48) (end 198.8983 78.23) (width 0.3) (layer "B.Cu") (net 12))
 (segment (start 198.8983 78.23) (end 196.0627 78.23) (width 0.3) (layer "B.Cu") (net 12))
 (segment (start 193.14 80.32) (end 196.5 76.96) (width 0.3) (layer "F.Cu") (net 11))
 (segment (start 190.5 80.32) (end 193.14 80.32) (width 0.3) (layer "F.Cu") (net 11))
 (segment (start 196.5 76.96) (end 200.68 72.78) (width 0.3) (layer "B.Cu") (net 11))
 (segment (start 200.68 72.78) (end 200.68 64) (width 0.3) (layer "B.Cu") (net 11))
 (segment (start 178 69.46) (end 179.27 70.73) (width 0.3) (layer "F.Cu") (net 10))
 (segment (start 197.7917 70.73) (end 203.22 65.3017) (width 0.3) (layer "F.Cu") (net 10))
 (segment (start 203.22 64) (end 203.22 65.3017) (width 0.3) (layer "F.Cu") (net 10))
 (segment (start 179.27 70.73) (end 197.7917 70.73) (width 0.3) (layer "F.Cu") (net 10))
 (segment (start 184 75.46) (end 178 69.46) (width 0.3) (layer "B.Cu") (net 10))
 (segment (start 184 80.32) (end 184 75.46) (width 0.3) (layer "B.Cu") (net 10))
 (segment (start 171.5 80.2167) (end 174.3233 80.2167) (width 0.3) (layer "F.Cu") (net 9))
 (segment (start 174.3233 80.2167) (end 177.5 77.04) (width 0.3) (layer "F.Cu") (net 9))
 (segment (start 212.361 71.9027) (end 205.76 65.3017) (width 0.3) (layer "B.Cu") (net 9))
 (segment (start 177.5 77.04) (end 183.468 83.008) (width 0.3) (layer "B.Cu") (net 9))
 (segment (start 183.468 83.008) (end 210.4864 83.008) (width 0.3) (layer "B.Cu") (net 9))
 (segment (start 205.76 64) (end 205.76 65.3017) (width 0.3) (layer "B.Cu") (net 9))
 (segment (start 212.361 81.1334) (end 212.361 71.9027) (width 0.3) (layer "B.Cu") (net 9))
 (segment (start 210.4864 83.008) (end 212.361 81.1334) (width 0.3) (layer "B.Cu") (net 9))
 (segment (start 220.8763 66.5) (end 222.3017 65.0746) (width 0.3) (layer "B.Cu") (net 45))
 (segment (start 222.3017 65.0746) (end 222.3017 62.9629) (width 0.3) (layer "B.Cu") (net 45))
 (segment (start 222.3017 62.9629) (end 221 61.6612) (width 0.3) (layer "B.Cu") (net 45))
 (segment (start 221 61.6612) (end 221 54) (width 0.3) (layer "B.Cu") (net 45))
 (segment (start 217 66.5) (end 220.8763 66.5) (width 0.3) (layer "B.Cu") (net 45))
 (segment (start 168.4237 64.2046) (end 168.4237 56.7063) (width 0.3) (layer "F.Cu") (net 43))
 (segment (start 177.4292 73.2101) (end 168.4237 64.2046) (width 0.3) (layer "F.Cu") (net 43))
 (segment (start 216.5 79) (end 216.5 77.7983) (width 0.3) (layer "F.Cu") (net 43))
 (segment (start 216.8755 77.7983) (end 217.7089 76.9649) (width 0.3) (layer "F.Cu") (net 43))
 (segment (start 168.4237 56.7063) (end 169.725 55.405) (width 0.3) (layer "F.Cu") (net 43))
 (segment (start 199.7567 73.2101) (end 177.4292 73.2101) (width 0.3) (layer "F.Cu") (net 43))
 (segment (start 217.0261 75.2583) (end 201.8049 75.2583) (width 0.3) (layer "F.Cu") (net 43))
 (segment (start 216.5 77.7983) (end 216.8755 77.7983) (width 0.3) (layer "F.Cu") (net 43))
 (segment (start 217.7089 76.9649) (end 217.7089 75.9411) (width 0.3) (layer "F.Cu") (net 43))
 (segment (start 169.725 54.1033) (end 169.725 55.405) (width 0.3) (layer "F.Cu") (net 43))
 (segment (start 217.7089 75.9411) (end 217.0261 75.2583) (width 0.3) (layer "F.Cu") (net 43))
 (segment (start 201.8049 75.2583) (end 199.7567 73.2101) (width 0.3) (layer "F.Cu") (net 43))
 (segment (start 197 66.92) (end 195.7983 66.92) (width 0.3) (layer "F.Cu") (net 42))
 (segment (start 170.5015 57.4227) (end 169.0288 58.8954) (width 0.3) (layer "F.Cu") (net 42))
 (segment (start 179.98 54.1033) (end 176.6606 57.4227) (width 0.3) (layer "F.Cu") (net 42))
 (segment (start 194.5283 68.19) (end 195.7983 66.92) (width 0.3) (layer "F.Cu") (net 42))
 (segment (start 176.6606 57.4227) (end 170.5015 57.4227) (width 0.3) (layer "F.Cu") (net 42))
 (segment (start 169.0288 60.9491) (end 176.2697 68.19) (width 0.3) (layer "F.Cu") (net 42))
 (segment (start 176.2697 68.19) (end 194.5283 68.19) (width 0.3) (layer "F.Cu") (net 42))
 (segment (start 169.0288 58.8954) (end 169.0288 60.9491) (width 0.3) (layer "F.Cu") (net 42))
 (segment (start 187.7913 56.547) (end 190.235 54.1033) (width 0.3) (layer "B.Cu") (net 41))
 (segment (start 173.9348 63.4003) (end 180.7881 56.547) (width 0.3) (layer "B.Cu") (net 41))
 (segment (start 180.7881 56.547) (end 187.7913 56.547) (width 0.3) (layer "B.Cu") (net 41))
 (segment (start 173.9348 64.4986) (end 173.9348 63.4003) (width 0.3) (layer "B.Cu") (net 41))
 (segment (start 178.9267 65.7071) (end 175.1433 65.7071) (width 0.3) (layer "B.Cu") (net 41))
 (segment (start 192.7196 79.5) (end 178.9267 65.7071) (width 0.3) (layer "B.Cu") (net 41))
 (segment (start 175.1433 65.7071) (end 173.9348 64.4986) (width 0.3) (layer "B.Cu") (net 41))
 (segment (start 196.5 79.5) (end 192.7196 79.5) (width 0.3) (layer "B.Cu") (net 41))
 (segment (start 169.6305 60.6999) (end 169.6305 59.1446) (width 0.3) (layer "F.Cu") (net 40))
 (segment (start 176.7983 66.92) (end 175.8506 66.92) (width 0.3) (layer "F.Cu") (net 40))
 (segment (start 178 66.92) (end 176.7983 66.92) (width 0.3) (layer "F.Cu") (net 40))
 (segment (start 196.5688 58.0245) (end 200.49 54.1033) (width 0.3) (layer "F.Cu") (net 40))
 (segment (start 175.8506 66.92) (end 169.6305 60.6999) (width 0.3) (layer "F.Cu") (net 40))
 (segment (start 169.6305 59.1446) (end 170.7506 58.0245) (width 0.3) (layer "F.Cu") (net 40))
 (segment (start 170.7506 58.0245) (end 196.5688 58.0245) (width 0.3) (layer "F.Cu") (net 40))
 (segment (start 169.6401 59.0864) (end 175.9374 52.7891) (width 0.3) (layer "B.Cu") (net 44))
 (segment (start 177.5 79.58) (end 177.5 78.3783) (width 0.3) (layer "B.Cu") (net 44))
 (segment (start 177.5 78.3783) (end 177.1245 78.3783) (width 0.3) (layer "B.Cu") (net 44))
 (segment (start 177.1245 78.3783) (end 169.6401 70.8939) (width 0.3) (layer "B.Cu") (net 44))
 (segment (start 169.6401 70.8939) (end 169.6401 59.0864) (width 0.3) (layer "B.Cu") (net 44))
 (segment (start 175.9374 52.7891) (end 209.4308 52.7891) (width 0.3) (layer "B.Cu") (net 44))
 (segment (start 209.4308 52.7891) (end 210.745 54.1033) (width 0.3) (layer "B.Cu") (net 44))
 (segment (start 217.4117 70.2736) (end 218.3395 71.2014) (width 0.3) (layer "F.Cu") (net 3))
 (segment (start 215.7542 69.547) (end 216.4808 70.2736) (width 0.3) (layer "F.Cu") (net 3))
 (segment (start 218.3395 71.2014) (end 218.3395 79.3397) (width 0.3) (layer "F.Cu") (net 3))
 (segment (start 218.3395 79.3397) (end 215.3259 82.3533) (width 0.3) (layer "F.Cu") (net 3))
 (segment (start 216.5786 67.7114) (end 215.7542 68.5358) (width 0.3) (layer "F.Cu") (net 3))
 (segment (start 221 65.3017) (end 218.5903 67.7114) (width 0.3) (layer "F.Cu") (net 3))
 (segment (start 164 81.765) (end 165.3017 81.765) (width 0.3) (layer "F.Cu") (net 3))
 (segment (start 215.7542 68.5358) (end 215.7542 69.547) (width 0.3) (layer "F.Cu") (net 3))
 (segment (start 218.5903 67.7114) (end 216.5786 67.7114) (width 0.3) (layer "F.Cu") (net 3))
 (segment (start 221 64) (end 221 65.3017) (width 0.3) (layer "F.Cu") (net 3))
 (segment (start 215.3259 82.3533) (end 165.89 82.3533) (width 0.3) (layer "F.Cu") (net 3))
 (segment (start 216.4808 70.2736) (end 217.4117 70.2736) (width 0.3) (layer "F.Cu") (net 3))
 (segment (start 165.89 82.3533) (end 165.3017 81.765) (width 0.3) (layer "F.Cu") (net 3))
 (segment (start 213.24 89.54) (end 215.92 86.86) (width 0.3) (layer "F.Cu") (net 23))
 (segment (start 170 89.54) (end 213.24 89.54) (width 0.3) (layer "F.Cu") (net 23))
 (segment (start 172.464 88.1623) (end 171.3017 87) (width 0.3) (layer "F.Cu") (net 26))
 (segment (start 206.9977 88.1623) (end 172.464 88.1623) (width 0.3) (layer "F.Cu") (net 26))
 (segment (start 208.3 86.86) (end 206.9977 88.1623) (width 0.3) (layer "F.Cu") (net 26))
 (segment (start 170 87) (end 171.3017 87) (width 0.3) (layer "F.Cu") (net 26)))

